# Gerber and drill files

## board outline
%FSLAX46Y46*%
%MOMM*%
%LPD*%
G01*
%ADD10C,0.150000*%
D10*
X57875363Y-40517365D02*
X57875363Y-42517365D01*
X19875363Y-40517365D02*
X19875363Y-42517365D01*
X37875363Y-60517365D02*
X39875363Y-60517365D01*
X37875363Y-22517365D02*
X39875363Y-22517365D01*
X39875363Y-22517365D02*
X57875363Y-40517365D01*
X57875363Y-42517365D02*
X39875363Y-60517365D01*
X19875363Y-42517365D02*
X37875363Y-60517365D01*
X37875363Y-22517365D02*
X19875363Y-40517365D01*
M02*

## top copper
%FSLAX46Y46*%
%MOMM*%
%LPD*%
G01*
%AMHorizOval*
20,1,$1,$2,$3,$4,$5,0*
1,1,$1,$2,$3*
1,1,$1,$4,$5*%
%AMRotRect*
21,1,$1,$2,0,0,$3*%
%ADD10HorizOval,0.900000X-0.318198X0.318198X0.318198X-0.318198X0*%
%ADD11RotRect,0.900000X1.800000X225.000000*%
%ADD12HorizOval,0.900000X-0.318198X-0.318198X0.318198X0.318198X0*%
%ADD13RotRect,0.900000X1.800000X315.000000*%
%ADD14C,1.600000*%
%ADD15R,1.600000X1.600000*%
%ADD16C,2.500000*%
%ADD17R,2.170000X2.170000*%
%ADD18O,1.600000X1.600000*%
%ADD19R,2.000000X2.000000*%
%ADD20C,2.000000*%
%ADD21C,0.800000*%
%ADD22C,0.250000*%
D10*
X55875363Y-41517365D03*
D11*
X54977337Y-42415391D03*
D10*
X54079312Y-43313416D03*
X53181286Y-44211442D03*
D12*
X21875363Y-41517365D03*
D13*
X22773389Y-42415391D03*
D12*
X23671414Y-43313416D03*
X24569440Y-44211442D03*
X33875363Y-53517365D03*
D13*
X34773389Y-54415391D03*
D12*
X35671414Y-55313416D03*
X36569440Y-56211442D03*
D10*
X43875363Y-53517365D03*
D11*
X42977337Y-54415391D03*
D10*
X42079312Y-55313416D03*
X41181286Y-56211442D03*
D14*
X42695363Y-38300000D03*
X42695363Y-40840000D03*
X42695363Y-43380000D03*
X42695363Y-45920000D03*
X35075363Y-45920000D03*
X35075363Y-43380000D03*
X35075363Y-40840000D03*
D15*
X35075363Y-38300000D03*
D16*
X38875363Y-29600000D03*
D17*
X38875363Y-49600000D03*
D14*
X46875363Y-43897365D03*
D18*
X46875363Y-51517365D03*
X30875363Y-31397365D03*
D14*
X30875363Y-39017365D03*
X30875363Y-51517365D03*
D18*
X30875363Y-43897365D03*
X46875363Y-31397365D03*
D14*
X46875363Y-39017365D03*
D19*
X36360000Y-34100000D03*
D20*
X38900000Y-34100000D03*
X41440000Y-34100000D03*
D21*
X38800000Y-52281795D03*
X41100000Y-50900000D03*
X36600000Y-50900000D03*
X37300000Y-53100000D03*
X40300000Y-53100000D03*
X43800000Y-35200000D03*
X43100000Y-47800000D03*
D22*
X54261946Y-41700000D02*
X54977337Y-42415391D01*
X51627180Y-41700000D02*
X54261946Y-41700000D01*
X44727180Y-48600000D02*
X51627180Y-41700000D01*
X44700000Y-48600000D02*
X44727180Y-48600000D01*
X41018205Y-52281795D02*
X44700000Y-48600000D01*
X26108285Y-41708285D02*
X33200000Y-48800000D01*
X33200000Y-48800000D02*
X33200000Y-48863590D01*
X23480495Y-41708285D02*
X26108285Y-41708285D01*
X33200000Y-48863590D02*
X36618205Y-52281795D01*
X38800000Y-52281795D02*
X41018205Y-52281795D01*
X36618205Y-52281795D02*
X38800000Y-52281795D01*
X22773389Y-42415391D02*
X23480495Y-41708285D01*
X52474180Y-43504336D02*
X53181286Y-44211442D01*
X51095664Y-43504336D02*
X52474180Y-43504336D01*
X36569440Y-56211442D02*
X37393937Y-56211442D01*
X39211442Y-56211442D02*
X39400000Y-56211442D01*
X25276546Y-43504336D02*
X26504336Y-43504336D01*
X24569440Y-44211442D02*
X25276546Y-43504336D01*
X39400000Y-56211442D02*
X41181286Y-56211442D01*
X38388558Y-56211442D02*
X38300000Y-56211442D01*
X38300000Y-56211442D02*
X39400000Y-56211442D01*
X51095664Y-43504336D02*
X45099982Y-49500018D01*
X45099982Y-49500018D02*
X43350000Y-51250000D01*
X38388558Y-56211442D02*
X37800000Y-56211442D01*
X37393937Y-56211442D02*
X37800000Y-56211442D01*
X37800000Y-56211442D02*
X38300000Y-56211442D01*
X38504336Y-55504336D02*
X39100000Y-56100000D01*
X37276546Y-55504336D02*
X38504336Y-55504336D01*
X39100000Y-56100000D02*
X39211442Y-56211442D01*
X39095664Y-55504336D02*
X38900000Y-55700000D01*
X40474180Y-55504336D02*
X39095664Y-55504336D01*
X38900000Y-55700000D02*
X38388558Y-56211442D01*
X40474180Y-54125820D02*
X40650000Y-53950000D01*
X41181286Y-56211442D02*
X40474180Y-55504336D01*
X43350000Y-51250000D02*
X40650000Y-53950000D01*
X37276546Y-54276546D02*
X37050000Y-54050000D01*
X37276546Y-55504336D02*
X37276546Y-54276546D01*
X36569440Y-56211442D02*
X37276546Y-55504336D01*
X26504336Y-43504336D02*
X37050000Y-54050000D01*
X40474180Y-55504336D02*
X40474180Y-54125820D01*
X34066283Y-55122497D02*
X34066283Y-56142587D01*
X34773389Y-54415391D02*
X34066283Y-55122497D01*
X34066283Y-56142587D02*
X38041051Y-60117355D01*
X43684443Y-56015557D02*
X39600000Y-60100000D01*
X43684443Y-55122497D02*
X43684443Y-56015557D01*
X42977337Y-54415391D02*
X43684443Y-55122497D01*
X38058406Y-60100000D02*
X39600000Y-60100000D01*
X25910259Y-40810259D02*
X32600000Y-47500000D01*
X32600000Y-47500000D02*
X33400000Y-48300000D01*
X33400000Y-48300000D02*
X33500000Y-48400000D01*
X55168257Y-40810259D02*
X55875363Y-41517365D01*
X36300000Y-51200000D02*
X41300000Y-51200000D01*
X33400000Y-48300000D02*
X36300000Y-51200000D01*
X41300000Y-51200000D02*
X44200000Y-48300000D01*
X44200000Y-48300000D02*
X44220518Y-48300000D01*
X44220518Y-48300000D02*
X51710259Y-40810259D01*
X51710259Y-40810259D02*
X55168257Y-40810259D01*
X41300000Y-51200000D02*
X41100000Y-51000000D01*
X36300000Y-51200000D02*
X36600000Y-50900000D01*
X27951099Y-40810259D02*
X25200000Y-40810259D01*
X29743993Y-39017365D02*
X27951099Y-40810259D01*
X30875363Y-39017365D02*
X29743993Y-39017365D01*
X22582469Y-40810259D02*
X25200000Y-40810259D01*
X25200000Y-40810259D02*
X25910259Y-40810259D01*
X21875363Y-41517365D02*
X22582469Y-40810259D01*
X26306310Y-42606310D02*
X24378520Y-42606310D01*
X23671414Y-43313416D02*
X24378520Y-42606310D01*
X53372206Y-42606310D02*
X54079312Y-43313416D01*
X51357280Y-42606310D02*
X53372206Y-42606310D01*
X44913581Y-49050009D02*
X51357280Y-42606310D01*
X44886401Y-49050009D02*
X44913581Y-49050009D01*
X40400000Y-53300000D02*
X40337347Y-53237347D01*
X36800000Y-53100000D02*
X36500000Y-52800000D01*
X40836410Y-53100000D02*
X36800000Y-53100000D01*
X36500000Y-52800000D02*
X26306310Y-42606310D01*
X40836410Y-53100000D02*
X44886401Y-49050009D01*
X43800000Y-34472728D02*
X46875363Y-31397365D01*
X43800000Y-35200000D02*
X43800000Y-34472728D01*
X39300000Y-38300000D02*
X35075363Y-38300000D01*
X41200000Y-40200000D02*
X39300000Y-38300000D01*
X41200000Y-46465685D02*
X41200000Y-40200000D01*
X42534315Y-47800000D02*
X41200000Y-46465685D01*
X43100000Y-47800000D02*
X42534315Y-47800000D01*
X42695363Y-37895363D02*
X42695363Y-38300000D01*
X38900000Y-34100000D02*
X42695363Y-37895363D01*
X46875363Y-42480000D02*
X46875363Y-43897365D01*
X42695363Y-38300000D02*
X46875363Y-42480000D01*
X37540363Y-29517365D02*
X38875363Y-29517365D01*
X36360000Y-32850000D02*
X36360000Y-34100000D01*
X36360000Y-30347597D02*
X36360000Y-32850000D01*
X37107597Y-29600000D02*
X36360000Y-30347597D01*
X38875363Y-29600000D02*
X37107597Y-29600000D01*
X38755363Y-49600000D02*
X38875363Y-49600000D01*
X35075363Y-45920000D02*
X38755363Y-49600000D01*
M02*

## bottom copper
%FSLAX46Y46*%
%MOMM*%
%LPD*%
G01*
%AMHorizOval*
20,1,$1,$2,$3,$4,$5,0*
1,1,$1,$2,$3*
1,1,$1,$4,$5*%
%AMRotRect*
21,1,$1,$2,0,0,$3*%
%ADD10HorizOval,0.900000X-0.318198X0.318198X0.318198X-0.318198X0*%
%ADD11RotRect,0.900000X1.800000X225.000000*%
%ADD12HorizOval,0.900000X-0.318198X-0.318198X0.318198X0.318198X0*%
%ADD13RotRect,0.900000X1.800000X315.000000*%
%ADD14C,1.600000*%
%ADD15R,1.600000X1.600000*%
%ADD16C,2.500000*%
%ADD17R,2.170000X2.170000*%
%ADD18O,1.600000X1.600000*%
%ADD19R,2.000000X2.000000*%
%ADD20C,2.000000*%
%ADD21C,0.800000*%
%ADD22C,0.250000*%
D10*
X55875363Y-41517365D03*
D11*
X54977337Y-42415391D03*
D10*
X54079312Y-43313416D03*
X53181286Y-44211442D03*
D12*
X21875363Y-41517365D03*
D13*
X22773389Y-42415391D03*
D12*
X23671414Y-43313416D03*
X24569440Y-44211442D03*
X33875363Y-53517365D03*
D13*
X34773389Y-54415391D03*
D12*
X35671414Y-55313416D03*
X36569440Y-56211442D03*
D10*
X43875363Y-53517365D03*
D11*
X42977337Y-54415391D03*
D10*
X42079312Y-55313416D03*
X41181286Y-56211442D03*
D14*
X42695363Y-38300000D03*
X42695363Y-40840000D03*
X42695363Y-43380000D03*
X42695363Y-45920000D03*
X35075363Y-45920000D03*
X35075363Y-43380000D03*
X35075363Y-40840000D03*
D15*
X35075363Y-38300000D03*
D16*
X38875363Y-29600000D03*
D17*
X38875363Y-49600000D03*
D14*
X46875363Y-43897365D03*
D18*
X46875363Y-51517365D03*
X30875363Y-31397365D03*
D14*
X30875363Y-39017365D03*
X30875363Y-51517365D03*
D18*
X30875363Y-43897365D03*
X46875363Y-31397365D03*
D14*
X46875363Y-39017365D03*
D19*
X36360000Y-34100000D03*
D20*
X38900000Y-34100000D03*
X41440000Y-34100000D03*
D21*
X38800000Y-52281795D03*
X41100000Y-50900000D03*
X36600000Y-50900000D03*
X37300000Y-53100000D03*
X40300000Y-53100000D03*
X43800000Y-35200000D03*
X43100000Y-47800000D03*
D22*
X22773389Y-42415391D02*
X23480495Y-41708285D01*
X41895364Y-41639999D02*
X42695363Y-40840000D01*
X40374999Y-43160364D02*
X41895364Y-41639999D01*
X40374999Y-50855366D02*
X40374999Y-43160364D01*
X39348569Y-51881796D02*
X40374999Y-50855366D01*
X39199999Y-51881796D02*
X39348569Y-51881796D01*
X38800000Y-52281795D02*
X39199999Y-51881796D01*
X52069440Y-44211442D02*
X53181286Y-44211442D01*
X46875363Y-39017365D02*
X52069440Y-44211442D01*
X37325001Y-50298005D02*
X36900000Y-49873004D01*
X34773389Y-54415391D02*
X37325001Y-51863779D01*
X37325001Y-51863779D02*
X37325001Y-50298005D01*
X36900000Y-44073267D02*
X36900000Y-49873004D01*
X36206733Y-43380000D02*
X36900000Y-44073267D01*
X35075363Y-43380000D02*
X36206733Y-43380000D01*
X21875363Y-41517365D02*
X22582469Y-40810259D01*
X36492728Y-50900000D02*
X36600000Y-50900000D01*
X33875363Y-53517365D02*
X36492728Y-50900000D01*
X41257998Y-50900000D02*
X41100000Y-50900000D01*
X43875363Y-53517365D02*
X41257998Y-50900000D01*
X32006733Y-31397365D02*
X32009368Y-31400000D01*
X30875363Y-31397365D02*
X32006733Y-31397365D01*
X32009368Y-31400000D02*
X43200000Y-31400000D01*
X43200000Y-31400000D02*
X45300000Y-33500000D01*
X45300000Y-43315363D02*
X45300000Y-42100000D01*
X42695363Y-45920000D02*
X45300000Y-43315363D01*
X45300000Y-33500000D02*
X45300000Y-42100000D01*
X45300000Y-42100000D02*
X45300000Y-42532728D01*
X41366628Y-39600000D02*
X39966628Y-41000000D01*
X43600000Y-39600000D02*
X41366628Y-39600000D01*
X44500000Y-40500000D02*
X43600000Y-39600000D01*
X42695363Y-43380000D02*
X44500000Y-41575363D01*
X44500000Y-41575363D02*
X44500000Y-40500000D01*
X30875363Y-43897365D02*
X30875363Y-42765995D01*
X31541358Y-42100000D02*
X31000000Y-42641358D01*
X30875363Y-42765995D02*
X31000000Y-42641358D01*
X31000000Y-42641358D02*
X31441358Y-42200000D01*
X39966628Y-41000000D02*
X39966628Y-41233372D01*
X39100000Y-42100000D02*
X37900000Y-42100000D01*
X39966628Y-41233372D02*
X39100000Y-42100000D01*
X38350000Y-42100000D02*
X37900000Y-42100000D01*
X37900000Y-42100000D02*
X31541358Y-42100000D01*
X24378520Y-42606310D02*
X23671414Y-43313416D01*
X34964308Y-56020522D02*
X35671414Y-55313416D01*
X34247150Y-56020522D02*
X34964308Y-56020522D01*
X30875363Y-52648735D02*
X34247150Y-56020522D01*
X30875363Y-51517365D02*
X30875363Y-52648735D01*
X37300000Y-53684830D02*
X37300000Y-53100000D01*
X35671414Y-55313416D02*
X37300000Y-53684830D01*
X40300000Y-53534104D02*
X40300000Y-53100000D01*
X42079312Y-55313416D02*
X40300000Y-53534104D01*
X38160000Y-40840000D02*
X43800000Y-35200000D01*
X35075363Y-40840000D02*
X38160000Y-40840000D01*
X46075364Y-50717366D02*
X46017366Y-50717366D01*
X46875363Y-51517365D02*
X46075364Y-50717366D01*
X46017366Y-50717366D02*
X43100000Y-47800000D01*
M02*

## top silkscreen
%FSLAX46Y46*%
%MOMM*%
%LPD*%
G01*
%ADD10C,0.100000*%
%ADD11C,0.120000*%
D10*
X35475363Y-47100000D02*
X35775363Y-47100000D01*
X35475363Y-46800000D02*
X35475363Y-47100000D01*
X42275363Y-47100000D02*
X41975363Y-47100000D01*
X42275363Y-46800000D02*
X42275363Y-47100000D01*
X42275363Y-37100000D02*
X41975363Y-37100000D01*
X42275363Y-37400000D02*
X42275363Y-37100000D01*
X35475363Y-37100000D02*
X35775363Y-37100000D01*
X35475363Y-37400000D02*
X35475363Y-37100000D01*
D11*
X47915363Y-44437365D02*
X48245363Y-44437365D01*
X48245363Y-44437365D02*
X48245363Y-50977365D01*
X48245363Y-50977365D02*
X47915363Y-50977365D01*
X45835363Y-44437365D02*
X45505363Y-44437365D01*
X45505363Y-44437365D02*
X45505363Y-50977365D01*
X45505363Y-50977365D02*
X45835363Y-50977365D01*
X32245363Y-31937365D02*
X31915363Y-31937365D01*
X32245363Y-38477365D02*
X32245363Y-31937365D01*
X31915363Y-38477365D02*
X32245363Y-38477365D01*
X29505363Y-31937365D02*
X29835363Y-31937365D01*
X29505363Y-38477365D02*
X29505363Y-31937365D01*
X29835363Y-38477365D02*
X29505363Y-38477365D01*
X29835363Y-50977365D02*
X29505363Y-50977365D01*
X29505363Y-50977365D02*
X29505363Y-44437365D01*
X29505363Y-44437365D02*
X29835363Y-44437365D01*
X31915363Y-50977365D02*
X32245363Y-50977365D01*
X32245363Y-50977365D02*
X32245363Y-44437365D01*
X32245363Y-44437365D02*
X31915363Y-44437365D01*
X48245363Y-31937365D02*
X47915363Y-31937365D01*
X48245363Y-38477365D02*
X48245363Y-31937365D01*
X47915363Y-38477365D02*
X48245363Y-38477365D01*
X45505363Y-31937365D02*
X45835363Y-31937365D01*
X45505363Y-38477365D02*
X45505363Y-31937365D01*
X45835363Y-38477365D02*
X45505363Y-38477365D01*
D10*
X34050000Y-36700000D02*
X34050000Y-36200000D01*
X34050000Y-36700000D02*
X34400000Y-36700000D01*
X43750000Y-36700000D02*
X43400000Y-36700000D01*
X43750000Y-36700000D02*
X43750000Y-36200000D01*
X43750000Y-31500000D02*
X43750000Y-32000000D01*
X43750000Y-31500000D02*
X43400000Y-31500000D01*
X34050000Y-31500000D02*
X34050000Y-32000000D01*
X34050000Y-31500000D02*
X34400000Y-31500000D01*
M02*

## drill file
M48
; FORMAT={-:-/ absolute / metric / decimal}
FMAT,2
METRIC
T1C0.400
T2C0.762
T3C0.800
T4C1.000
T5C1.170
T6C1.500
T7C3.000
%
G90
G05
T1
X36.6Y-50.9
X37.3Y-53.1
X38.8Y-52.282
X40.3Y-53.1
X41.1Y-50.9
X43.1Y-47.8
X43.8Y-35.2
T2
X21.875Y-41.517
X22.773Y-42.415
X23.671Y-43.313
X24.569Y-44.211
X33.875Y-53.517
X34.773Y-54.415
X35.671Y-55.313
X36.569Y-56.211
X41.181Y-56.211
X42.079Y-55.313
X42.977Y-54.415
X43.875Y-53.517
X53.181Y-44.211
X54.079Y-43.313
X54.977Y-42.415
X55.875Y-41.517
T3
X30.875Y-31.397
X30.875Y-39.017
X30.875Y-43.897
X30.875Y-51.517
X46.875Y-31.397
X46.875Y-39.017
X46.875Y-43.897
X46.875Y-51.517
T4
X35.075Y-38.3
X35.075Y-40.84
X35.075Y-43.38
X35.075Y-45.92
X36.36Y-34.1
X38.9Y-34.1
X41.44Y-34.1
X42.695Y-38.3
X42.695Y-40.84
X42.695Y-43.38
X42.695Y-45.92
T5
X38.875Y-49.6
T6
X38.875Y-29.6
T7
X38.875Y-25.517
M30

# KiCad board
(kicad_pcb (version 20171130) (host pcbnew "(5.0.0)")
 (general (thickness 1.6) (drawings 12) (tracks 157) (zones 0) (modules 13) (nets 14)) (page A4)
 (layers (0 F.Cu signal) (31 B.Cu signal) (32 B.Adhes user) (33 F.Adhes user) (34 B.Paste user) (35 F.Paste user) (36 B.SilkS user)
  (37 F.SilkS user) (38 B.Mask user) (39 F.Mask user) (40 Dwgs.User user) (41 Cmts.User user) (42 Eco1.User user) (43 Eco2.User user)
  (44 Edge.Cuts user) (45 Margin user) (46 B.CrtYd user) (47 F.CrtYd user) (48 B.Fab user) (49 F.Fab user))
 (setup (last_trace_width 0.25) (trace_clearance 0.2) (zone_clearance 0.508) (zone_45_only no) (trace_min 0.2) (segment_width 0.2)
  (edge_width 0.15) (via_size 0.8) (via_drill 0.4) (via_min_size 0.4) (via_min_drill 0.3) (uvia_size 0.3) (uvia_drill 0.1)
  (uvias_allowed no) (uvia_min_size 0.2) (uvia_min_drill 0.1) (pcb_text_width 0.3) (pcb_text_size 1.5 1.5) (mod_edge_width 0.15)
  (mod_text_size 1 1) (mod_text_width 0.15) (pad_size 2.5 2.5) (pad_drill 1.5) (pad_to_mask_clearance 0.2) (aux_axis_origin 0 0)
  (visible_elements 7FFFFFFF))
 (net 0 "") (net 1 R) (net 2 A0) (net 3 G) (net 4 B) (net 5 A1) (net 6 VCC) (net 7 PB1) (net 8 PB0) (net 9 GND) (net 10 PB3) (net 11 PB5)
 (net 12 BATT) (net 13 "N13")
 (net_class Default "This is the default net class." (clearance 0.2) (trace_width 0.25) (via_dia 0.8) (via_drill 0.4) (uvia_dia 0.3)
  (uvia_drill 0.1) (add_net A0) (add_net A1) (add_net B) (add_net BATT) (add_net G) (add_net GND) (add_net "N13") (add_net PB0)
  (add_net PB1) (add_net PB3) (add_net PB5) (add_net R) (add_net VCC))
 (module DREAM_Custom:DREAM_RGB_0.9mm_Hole (layer F.Cu) (at 55.875363 41.517365 225)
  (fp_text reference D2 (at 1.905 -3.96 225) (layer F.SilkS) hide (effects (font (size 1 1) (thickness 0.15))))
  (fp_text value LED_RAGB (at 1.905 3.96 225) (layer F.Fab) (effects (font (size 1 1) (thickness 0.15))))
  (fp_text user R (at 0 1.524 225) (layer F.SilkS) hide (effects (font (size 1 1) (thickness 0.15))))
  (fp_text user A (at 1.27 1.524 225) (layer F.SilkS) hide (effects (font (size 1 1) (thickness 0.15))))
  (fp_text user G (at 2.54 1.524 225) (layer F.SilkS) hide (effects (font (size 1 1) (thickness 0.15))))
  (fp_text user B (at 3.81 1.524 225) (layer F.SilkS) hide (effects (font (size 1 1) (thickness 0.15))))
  (pad 1 thru_hole oval (at 0 0 225) (size 0.9 1.8) (drill 0.762) (layers *.Cu *.Mask) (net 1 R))
  (pad 2 thru_hole rect (at 1.270001 0 225) (size 0.9 1.8) (drill 0.762) (layers *.Cu *.Mask) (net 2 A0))
  (pad 3 thru_hole oval (at 2.54 0 225) (size 0.9 1.8) (drill 0.762) (layers *.Cu *.Mask) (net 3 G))
  (pad 4 thru_hole oval (at 3.81 0 225) (size 0.9 1.8) (drill 0.762) (layers *.Cu *.Mask) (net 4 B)))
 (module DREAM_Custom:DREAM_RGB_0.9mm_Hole (layer F.Cu) (at 21.875363 41.517365 315)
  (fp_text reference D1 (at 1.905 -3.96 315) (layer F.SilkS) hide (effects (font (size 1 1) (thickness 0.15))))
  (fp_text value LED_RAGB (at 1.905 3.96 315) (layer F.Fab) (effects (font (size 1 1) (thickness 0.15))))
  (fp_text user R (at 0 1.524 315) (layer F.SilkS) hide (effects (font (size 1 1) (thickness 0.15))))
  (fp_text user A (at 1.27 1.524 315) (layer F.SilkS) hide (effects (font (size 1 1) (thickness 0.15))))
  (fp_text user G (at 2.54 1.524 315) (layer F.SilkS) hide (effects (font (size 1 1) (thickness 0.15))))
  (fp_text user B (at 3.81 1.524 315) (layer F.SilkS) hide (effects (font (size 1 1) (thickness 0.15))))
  (pad 1 thru_hole oval (at 0 0 315) (size 0.9 1.8) (drill 0.762) (layers *.Cu *.Mask) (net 1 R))
  (pad 2 thru_hole rect (at 1.270001 0 315) (size 0.9 1.8) (drill 0.762) (layers *.Cu *.Mask) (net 2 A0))
  (pad 3 thru_hole oval (at 2.54 0 315) (size 0.9 1.8) (drill 0.762) (layers *.Cu *.Mask) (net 3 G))
  (pad 4 thru_hole oval (at 3.81 0 315) (size 0.9 1.8) (drill 0.762) (layers *.Cu *.Mask) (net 4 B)))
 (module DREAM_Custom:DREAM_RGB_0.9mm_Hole (layer F.Cu) (at 33.875363 53.517365 315)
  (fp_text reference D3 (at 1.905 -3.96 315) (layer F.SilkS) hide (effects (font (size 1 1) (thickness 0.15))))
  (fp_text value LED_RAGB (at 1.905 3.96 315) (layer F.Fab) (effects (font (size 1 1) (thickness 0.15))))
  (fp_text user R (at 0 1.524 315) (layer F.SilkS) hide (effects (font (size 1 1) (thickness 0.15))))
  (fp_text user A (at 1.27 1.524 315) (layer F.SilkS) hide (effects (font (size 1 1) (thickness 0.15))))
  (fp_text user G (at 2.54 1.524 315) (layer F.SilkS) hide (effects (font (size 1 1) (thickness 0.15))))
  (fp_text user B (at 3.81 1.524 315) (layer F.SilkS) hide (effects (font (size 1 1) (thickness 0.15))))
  (pad 1 thru_hole oval (at 0 0 315) (size 0.9 1.8) (drill 0.762) (layers *.Cu *.Mask) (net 1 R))
  (pad 2 thru_hole rect (at 1.270001 0 315) (size 0.9 1.8) (drill 0.762) (layers *.Cu *.Mask) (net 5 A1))
  (pad 3 thru_hole oval (at 2.54 0 315) (size 0.9 1.8) (drill 0.762) (layers *.Cu *.Mask) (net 3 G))
  (pad 4 thru_hole oval (at 3.81 0 315) (size 0.9 1.8) (drill 0.762) (layers *.Cu *.Mask) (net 4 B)))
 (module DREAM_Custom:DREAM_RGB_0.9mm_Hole (layer F.Cu) (at 43.875363 53.517365 225)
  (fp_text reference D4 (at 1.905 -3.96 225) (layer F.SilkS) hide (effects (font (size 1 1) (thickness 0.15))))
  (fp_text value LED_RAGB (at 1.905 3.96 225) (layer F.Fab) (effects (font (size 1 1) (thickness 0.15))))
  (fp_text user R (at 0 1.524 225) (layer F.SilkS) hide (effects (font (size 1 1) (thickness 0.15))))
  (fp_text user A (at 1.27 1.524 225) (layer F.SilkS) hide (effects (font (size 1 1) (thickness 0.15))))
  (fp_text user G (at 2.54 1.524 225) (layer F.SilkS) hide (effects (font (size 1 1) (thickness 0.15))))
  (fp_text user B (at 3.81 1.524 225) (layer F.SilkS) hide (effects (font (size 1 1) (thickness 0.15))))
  (pad 1 thru_hole oval (at 0 0 225) (size 0.9 1.8) (drill 0.762) (layers *.Cu *.Mask) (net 1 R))
  (pad 2 thru_hole rect (at 1.270001 0 225) (size 0.9 1.8) (drill 0.762) (layers *.Cu *.Mask) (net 5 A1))
  (pad 3 thru_hole oval (at 2.54 0 225) (size 0.9 1.8) (drill 0.762) (layers *.Cu *.Mask) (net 3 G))
  (pad 4 thru_hole oval (at 3.81 0 225) (size 0.9 1.8) (drill 0.762) (layers *.Cu *.Mask) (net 4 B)))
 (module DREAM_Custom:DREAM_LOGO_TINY (layer B.Cu) (at 38.9 40.65 180)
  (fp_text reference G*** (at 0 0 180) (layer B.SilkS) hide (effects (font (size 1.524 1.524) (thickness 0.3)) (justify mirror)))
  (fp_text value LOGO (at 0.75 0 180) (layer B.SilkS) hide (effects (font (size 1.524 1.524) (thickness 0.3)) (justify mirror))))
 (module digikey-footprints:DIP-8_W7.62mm (layer F.Cu) (at 35.075363 38.3)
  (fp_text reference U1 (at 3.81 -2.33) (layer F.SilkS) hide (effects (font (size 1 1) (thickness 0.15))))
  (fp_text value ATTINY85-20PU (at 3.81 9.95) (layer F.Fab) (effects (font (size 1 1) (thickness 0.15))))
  (fp_line (start 0.4 8.8) (end 0.7 8.8) (layer F.SilkS) (width 0.1))
  (fp_line (start 0.4 8.5) (end 0.4 8.8) (layer F.SilkS) (width 0.1))
  (fp_line (start 7.2 8.8) (end 6.9 8.8) (layer F.SilkS) (width 0.1))
  (fp_line (start 7.2 8.5) (end 7.2 8.8) (layer F.SilkS) (width 0.1))
  (fp_line (start 7.2 -1.2) (end 6.9 -1.2) (layer F.SilkS) (width 0.1))
  (fp_line (start 7.2 -0.9) (end 7.2 -1.2) (layer F.SilkS) (width 0.1))
  (fp_line (start 0.4 -1.2) (end 0.7 -1.2) (layer F.SilkS) (width 0.1))
  (fp_line (start 0.4 -0.9) (end 0.4 -1.2) (layer F.SilkS) (width 0.1))
  (pad 8 thru_hole circle (at 7.62 0) (size 1.6 1.6) (drill 1) (layers *.Cu *.Mask) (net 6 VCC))
  (pad 7 thru_hole circle (at 7.62 2.54) (size 1.6 1.6) (drill 1) (layers *.Cu *.Mask) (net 2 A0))
  (pad 6 thru_hole circle (at 7.62 5.08) (size 1.6 1.6) (drill 1) (layers *.Cu *.Mask) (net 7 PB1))
  (pad 5 thru_hole circle (at 7.62 7.62) (size 1.6 1.6) (drill 1) (layers *.Cu *.Mask) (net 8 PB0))
  (pad 4 thru_hole circle (at 0 7.62) (size 1.6 1.6) (drill 1) (layers *.Cu *.Mask) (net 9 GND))
  (pad 3 thru_hole circle (at 0 5.08) (size 1.6 1.6) (drill 1) (layers *.Cu *.Mask) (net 5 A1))
  (pad 2 thru_hole circle (at 0 2.54) (size 1.6 1.6) (drill 1) (layers *.Cu *.Mask) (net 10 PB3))
  (pad 1 thru_hole rect (at 0 0) (size 1.6 1.6) (drill 1) (layers *.Cu *.Mask) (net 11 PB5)))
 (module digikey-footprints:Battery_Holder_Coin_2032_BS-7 (layer B.Cu) (at 38.875363 49.6 90)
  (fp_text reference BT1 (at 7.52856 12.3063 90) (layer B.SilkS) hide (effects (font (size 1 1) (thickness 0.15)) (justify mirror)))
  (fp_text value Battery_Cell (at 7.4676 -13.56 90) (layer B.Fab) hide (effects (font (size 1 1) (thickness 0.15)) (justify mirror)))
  (pad Pos thru_hole circle (at 20 0 90) (size 2.5 2.5) (drill 1.5) (layers *.Cu *.Mask) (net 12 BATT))
  (pad Neg thru_hole rect (at 0 0 90) (size 2.17 2.17) (drill 1.17) (layers *.Cu *.Mask) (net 9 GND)))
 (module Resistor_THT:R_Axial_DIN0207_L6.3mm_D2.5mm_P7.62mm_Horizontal (layer F.Cu) (at 46.875363 43.897365 270)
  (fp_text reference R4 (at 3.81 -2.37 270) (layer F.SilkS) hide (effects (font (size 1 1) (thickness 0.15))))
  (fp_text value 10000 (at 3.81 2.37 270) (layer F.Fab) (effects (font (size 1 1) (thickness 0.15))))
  (fp_line (start 0.54 -1.04) (end 0.54 -1.37) (layer F.SilkS) (width 0.12))
  (fp_line (start 0.54 -1.37) (end 7.08 -1.37) (layer F.SilkS) (width 0.12))
  (fp_line (start 7.08 -1.37) (end 7.08 -1.04) (layer F.SilkS) (width 0.12))
  (fp_line (start 0.54 1.04) (end 0.54 1.37) (layer F.SilkS) (width 0.12))
  (fp_line (start 0.54 1.37) (end 7.08 1.37) (layer F.SilkS) (width 0.12))
  (fp_line (start 7.08 1.37) (end 7.08 1.04) (layer F.SilkS) (width 0.12))
  (pad 1 thru_hole circle (at 0 0 270) (size 1.6 1.6) (drill 0.8) (layers *.Cu *.Mask) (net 6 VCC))
  (pad 2 thru_hole oval (at 7.62 0 270) (size 1.6 1.6) (drill 0.8) (layers *.Cu *.Mask) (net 11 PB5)))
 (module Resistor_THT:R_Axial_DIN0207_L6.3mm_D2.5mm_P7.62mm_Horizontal (layer F.Cu) (at 30.875363 39.017365 90)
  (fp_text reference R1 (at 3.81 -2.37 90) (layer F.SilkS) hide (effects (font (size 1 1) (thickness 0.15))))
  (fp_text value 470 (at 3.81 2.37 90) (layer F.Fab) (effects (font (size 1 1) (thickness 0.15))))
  (fp_line (start 7.08 1.37) (end 7.08 1.04) (layer F.SilkS) (width 0.12))
  (fp_line (start 0.54 1.37) (end 7.08 1.37) (layer F.SilkS) (width 0.12))
  (fp_line (start 0.54 1.04) (end 0.54 1.37) (layer F.SilkS) (width 0.12))
  (fp_line (start 7.08 -1.37) (end 7.08 -1.04) (layer F.SilkS) (width 0.12))
  (fp_line (start 0.54 -1.37) (end 7.08 -1.37) (layer F.SilkS) (width 0.12))
  (fp_line (start 0.54 -1.04) (end 0.54 -1.37) (layer F.SilkS) (width 0.12))
  (pad 2 thru_hole oval (at 7.62 0 90) (size 1.6 1.6) (drill 0.8) (layers *.Cu *.Mask) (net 8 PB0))
  (pad 1 thru_hole circle (at 0 0 90) (size 1.6 1.6) (drill 0.8) (layers *.Cu *.Mask) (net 1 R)))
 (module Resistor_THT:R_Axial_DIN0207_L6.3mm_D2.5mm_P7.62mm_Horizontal (layer F.Cu) (at 30.875363 51.517365 90)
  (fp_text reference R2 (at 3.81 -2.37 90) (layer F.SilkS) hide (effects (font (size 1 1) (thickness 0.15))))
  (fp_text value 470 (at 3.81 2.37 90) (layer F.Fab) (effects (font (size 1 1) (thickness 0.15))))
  (fp_line (start 0.54 -1.04) (end 0.54 -1.37) (layer F.SilkS) (width 0.12))
  (fp_line (start 0.54 -1.37) (end 7.08 -1.37) (layer F.SilkS) (width 0.12))
  (fp_line (start 7.08 -1.37) (end 7.08 -1.04) (layer F.SilkS) (width 0.12))
  (fp_line (start 0.54 1.04) (end 0.54 1.37) (layer F.SilkS) (width 0.12))
  (fp_line (start 0.54 1.37) (end 7.08 1.37) (layer F.SilkS) (width 0.12))
  (fp_line (start 7.08 1.37) (end 7.08 1.04) (layer F.SilkS) (width 0.12))
  (pad 1 thru_hole circle (at 0 0 90) (size 1.6 1.6) (drill 0.8) (layers *.Cu *.Mask) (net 3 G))
  (pad 2 thru_hole oval (at 7.62 0 90) (size 1.6 1.6) (drill 0.8) (layers *.Cu *.Mask) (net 7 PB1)))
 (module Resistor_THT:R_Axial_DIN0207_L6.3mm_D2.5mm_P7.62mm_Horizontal (layer F.Cu) (at 46.875363 39.017365 90)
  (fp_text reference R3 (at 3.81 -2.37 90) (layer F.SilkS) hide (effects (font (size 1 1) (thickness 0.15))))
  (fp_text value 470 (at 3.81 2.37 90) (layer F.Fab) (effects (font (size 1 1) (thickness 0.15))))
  (fp_line (start 7.08 1.37) (end 7.08 1.04) (layer F.SilkS) (width 0.12))
  (fp_line (start 0.54 1.37) (end 7.08 1.37) (layer F.SilkS) (width 0.12))
  (fp_line (start 0.54 1.04) (end 0.54 1.37) (layer F.SilkS) (width 0.12))
  (fp_line (start 7.08 -1.37) (end 7.08 -1.04) (layer F.SilkS) (width 0.12))
  (fp_line (start 0.54 -1.37) (end 7.08 -1.37) (layer F.SilkS) (width 0.12))
  (fp_line (start 0.54 -1.04) (end 0.54 -1.37) (layer F.SilkS) (width 0.12))
  (pad 2 thru_hole oval (at 7.62 0 90) (size 1.6 1.6) (drill 0.8) (layers *.Cu *.Mask) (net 10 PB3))
  (pad 1 thru_hole circle (at 0 0 90) (size 1.6 1.6) (drill 0.8) (layers *.Cu *.Mask) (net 4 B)))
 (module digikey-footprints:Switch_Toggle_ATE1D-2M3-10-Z (layer F.Cu) (at 38.9 34.1)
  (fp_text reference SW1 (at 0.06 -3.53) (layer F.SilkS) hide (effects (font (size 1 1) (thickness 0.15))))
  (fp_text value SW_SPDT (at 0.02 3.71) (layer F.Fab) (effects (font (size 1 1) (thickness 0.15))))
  (fp_line (start -4.85 2.6) (end -4.85 2.1) (layer F.SilkS) (width 0.1))
  (fp_line (start -4.85 2.6) (end -4.5 2.6) (layer F.SilkS) (width 0.1))
  (fp_line (start 4.85 2.6) (end 4.5 2.6) (layer F.SilkS) (width 0.1))
  (fp_line (start 4.85 2.6) (end 4.85 2.1) (layer F.SilkS) (width 0.1))
  (fp_line (start 4.85 -2.6) (end 4.85 -2.1) (layer F.SilkS) (width 0.1))
  (fp_line (start 4.85 -2.6) (end 4.5 -2.6) (layer F.SilkS) (width 0.1))
  (fp_line (start -4.85 -2.6) (end -4.85 -2.1) (layer F.SilkS) (width 0.1))
  (fp_line (start -4.85 -2.6) (end -4.5 -2.6) (layer F.SilkS) (width 0.1))
  (pad 1 thru_hole rect (at -2.54 0) (size 2 2) (drill 1) (layers *.Cu *.Mask) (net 12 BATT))
  (pad 2 thru_hole circle (at 0 0) (size 2 2) (drill 1) (layers *.Cu *.Mask) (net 6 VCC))
  (pad 3 thru_hole circle (at 2.54 0) (size 2 2) (drill 1) (layers *.Cu *.Mask) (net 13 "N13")))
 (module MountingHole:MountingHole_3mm (layer F.Cu) (at 38.875363 25.517365)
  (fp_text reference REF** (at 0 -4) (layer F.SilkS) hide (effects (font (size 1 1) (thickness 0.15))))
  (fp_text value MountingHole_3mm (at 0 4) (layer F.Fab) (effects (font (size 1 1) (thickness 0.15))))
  (pad 1 np_thru_hole circle (at 0 0) (size 3 3) (drill 3) (layers *.Cu *.Mask)))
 (gr_line (start 57.875363 40.517365) (end 57.875363 42.517365) (layer Edge.Cuts) (width 0.15))
 (gr_line (start 19.875363 40.517365) (end 19.875363 42.517365) (layer Edge.Cuts) (width 0.15))
 (gr_line (start 37.875363 60.517365) (end 39.875363 60.517365) (layer Edge.Cuts) (width 0.15))
 (gr_line (start 37.875363 22.517365) (end 39.875363 22.517365) (layer Edge.Cuts) (width 0.15))
 (gr_line (start 39.875363 22.517365) (end 57.875363 40.517365) (layer Edge.Cuts) (width 0.15))
 (gr_line (start 57.875363 42.517365) (end 39.875363 60.517365) (layer Edge.Cuts) (width 0.15))
 (gr_line (start 19.875363 42.517365) (end 37.875363 60.517365) (layer Edge.Cuts) (width 0.15))
 (gr_line (start 37.875363 22.517365) (end 19.875363 40.517365) (layer Edge.Cuts) (width 0.15))
 (segment (start 54.261946 41.7) (end 54.977337 42.415391) (width 0.25) (layer F.Cu) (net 2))
 (segment (start 51.62718 41.7) (end 54.261946 41.7) (width 0.25) (layer F.Cu) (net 2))
 (segment (start 44.72718 48.6) (end 51.62718 41.7) (width 0.25) (layer F.Cu) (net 2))
 (segment (start 44.7 48.6) (end 44.72718 48.6) (width 0.25) (layer F.Cu) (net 2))
 (segment (start 41.018205 52.281795) (end 44.7 48.6) (width 0.25) (layer F.Cu) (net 2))
 (segment (start 22.773389 42.415391) (end 23.480495 41.708285) (width 0.25) (layer B.Cu) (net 2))
 (segment (start 26.108285 41.708285) (end 33.2 48.8) (width 0.25) (layer F.Cu) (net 2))
 (segment (start 33.2 48.8) (end 33.2 48.86359) (width 0.25) (layer F.Cu) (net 2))
 (segment (start 23.480495 41.708285) (end 26.108285 41.708285) (width 0.25) (layer F.Cu) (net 2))
 (segment (start 33.2 48.86359) (end 36.618205 52.281795) (width 0.25) (layer F.Cu) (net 2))
 (via (at 38.8 52.281795) (size 0.8) (drill 0.4) (layers F.Cu B.Cu) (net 2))
 (segment (start 38.8 52.281795) (end 41.018205 52.281795) (width 0.25) (layer F.Cu) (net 2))
 (segment (start 36.618205 52.281795) (end 38.8 52.281795) (width 0.25) (layer F.Cu) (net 2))
 (segment (start 22.773389 42.415391) (end 23.480495 41.708285) (width 0.25) (layer F.Cu) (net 2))
 (segment (start 41.895364 41.639999) (end 42.695363 40.84) (width 0.25) (layer B.Cu) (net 2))
 (segment (start 40.374999 43.160364) (end 41.895364 41.639999) (width 0.25) (layer B.Cu) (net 2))
 (segment (start 40.374999 50.855366) (end 40.374999 43.160364) (width 0.25) (layer B.Cu) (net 2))
 (segment (start 39.348569 51.881796) (end 40.374999 50.855366) (width 0.25) (layer B.Cu) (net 2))
 (segment (start 39.199999 51.881796) (end 39.348569 51.881796) (width 0.25) (layer B.Cu) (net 2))
 (segment (start 38.8 52.281795) (end 39.199999 51.881796) (width 0.25) (layer B.Cu) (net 2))
 (segment (start 52.06944 44.211442) (end 53.181286 44.211442) (width 0.25) (layer B.Cu) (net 4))
 (segment (start 46.875363 39.017365) (end 52.06944 44.211442) (width 0.25) (layer B.Cu) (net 4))
 (segment (start 52.47418 43.504336) (end 53.181286 44.211442) (width 0.25) (layer F.Cu) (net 4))
 (segment (start 51.095664 43.504336) (end 52.47418 43.504336) (width 0.25) (layer F.Cu) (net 4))
 (segment (start 36.56944 56.211442) (end 37.393937 56.211442) (width 0.25) (layer F.Cu) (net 4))
 (segment (start 39.211442 56.211442) (end 39.4 56.211442) (width 0.25) (layer F.Cu) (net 4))
 (segment (start 25.276546 43.504336) (end 26.504336 43.504336) (width 0.25) (layer F.Cu) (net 4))
 (segment (start 24.56944 44.211442) (end 25.276546 43.504336) (width 0.25) (layer F.Cu) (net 4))
 (segment (start 39.4 56.211442) (end 41.181286 56.211442) (width 0.25) (layer F.Cu) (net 4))
 (segment (start 38.388558 56.211442) (end 38.3 56.211442) (width 0.25) (layer F.Cu) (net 4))
 (segment (start 38.3 56.211442) (end 39.4 56.211442) (width 0.25) (layer F.Cu) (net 4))
 (segment (start 51.095664 43.504336) (end 45.099982 49.500018) (width 0.25) (layer F.Cu) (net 4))
 (segment (start 45.099982 49.500018) (end 43.35 51.25) (width 0.25) (layer F.Cu) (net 4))
 (segment (start 38.388558 56.211442) (end 37.8 56.211442) (width 0.25) (layer F.Cu) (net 4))
 (segment (start 37.393937 56.211442) (end 37.8 56.211442) (width 0.25) (layer F.Cu) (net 4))
 (segment (start 37.8 56.211442) (end 38.3 56.211442) (width 0.25) (layer F.Cu) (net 4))
 (segment (start 38.504336 55.504336) (end 39.1 56.1) (width 0.25) (layer F.Cu) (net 4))
 (segment (start 37.276546 55.504336) (end 38.504336 55.504336) (width 0.25) (layer F.Cu) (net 4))
 (segment (start 39.1 56.1) (end 39.211442 56.211442) (width 0.25) (layer F.Cu) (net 4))
 (segment (start 39.095664 55.504336) (end 38.9 55.7) (width 0.25) (layer F.Cu) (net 4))
 (segment (start 40.47418 55.504336) (end 39.095664 55.504336) (width 0.25) (layer F.Cu) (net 4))
 (segment (start 38.9 55.7) (end 38.388558 56.211442) (width 0.25) (layer F.Cu) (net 4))
 (segment (start 40.47418 54.12582) (end 40.65 53.95) (width 0.25) (layer F.Cu) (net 4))
 (segment (start 41.181286 56.211442) (end 40.47418 55.504336) (width 0.25) (layer F.Cu) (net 4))
 (segment (start 43.35 51.25) (end 40.65 53.95) (width 0.25) (layer F.Cu) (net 4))
 (segment (start 37.276546 54.276546) (end 37.05 54.05) (width 0.25) (layer F.Cu) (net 4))
 (segment (start 37.276546 55.504336) (end 37.276546 54.276546) (width 0.25) (layer F.Cu) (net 4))
 (segment (start 36.56944 56.211442) (end 37.276546 55.504336) (width 0.25) (layer F.Cu) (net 4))
 (segment (start 26.504336 43.504336) (end 37.05 54.05) (width 0.25) (layer F.Cu) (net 4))
 (segment (start 40.47418 55.504336) (end 40.47418 54.12582) (width 0.25) (layer F.Cu) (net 4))
 (segment (start 34.066283 55.122497) (end 34.066283 56.142587) (width 0.25) (layer F.Cu) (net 5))
 (segment (start 34.773389 54.415391) (end 34.066283 55.122497) (width 0.25) (layer F.Cu) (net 5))
 (segment (start 34.066283 56.142587) (end 38.041051 60.117355) (width 0.25) (layer F.Cu) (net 5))
 (segment (start 43.684443 56.015557) (end 39.6 60.1) (width 0.25) (layer F.Cu) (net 5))
 (segment (start 43.684443 55.122497) (end 43.684443 56.015557) (width 0.25) (layer F.Cu) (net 5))
 (segment (start 42.977337 54.415391) (end 43.684443 55.122497) (width 0.25) (layer F.Cu) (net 5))
 (segment (start 38.058406 60.1) (end 39.6 60.1) (width 0.25) (layer F.Cu) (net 5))
 (segment (start 37.325001 50.298005) (end 36.9 49.873004) (width 0.25) (layer B.Cu) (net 5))
 (segment (start 34.773389 54.415391) (end 37.325001 51.863779) (width 0.25) (layer B.Cu) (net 5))
 (segment (start 37.325001 51.863779) (end 37.325001 50.298005) (width 0.25) (layer B.Cu) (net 5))
 (segment (start 36.9 44.073267) (end 36.9 49.873004) (width 0.25) (layer B.Cu) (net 5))
 (segment (start 36.206733 43.38) (end 36.9 44.073267) (width 0.25) (layer B.Cu) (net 5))
 (segment (start 35.075363 43.38) (end 36.206733 43.38) (width 0.25) (layer B.Cu) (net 5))
 (segment (start 21.875363 41.517365) (end 22.582469 40.810259) (width 0.25) (layer B.Cu) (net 1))
 (segment (start 25.910259 40.810259) (end 32.6 47.5) (width 0.25) (layer F.Cu) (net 1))
 (segment (start 32.6 47.5) (end 33.4 48.3) (width 0.25) (layer F.Cu) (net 1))
 (segment (start 33.4 48.3) (end 33.5 48.4) (width 0.25) (layer F.Cu) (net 1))
 (segment (start 55.168257 40.810259) (end 55.875363 41.517365) (width 0.25) (layer F.Cu) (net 1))
 (segment (start 36.3 51.2) (end 41.3 51.2) (width 0.25) (layer F.Cu) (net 1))
 (segment (start 33.4 48.3) (end 36.3 51.2) (width 0.25) (layer F.Cu) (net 1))
 (segment (start 41.3 51.2) (end 44.2 48.3) (width 0.25) (layer F.Cu) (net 1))
 (segment (start 44.2 48.3) (end 44.220518 48.3) (width 0.25) (layer F.Cu) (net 1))
 (segment (start 44.220518 48.3) (end 51.710259 40.810259) (width 0.25) (layer F.Cu) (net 1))
 (segment (start 51.710259 40.810259) (end 55.168257 40.810259) (width 0.25) (layer F.Cu) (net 1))
 (via (at 41.1 50.9) (size 0.8) (drill 0.4) (layers F.Cu B.Cu) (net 1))
 (segment (start 41.3 51.2) (end 41.1 51) (width 0.25) (layer F.Cu) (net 1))
 (via (at 36.6 50.9) (size 0.8) (drill 0.4) (layers F.Cu B.Cu) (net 1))
 (segment (start 36.3 51.2) (end 36.6 50.9) (width 0.25) (layer F.Cu) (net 1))
 (segment (start 36.492728 50.9) (end 36.6 50.9) (width 0.25) (layer B.Cu) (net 1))
 (segment (start 33.875363 53.517365) (end 36.492728 50.9) (width 0.25) (layer B.Cu) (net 1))
 (segment (start 41.257998 50.9) (end 41.1 50.9) (width 0.25) (layer B.Cu) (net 1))
 (segment (start 43.875363 53.517365) (end 41.257998 50.9) (width 0.25) (layer B.Cu) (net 1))
 (segment (start 27.951099 40.810259) (end 25.2 40.810259) (width 0.25) (layer F.Cu) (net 1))
 (segment (start 29.743993 39.017365) (end 27.951099 40.810259) (width 0.25) (layer F.Cu) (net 1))
 (segment (start 30.875363 39.017365) (end 29.743993 39.017365) (width 0.25) (layer F.Cu) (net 1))
 (segment (start 22.582469 40.810259) (end 25.2 40.810259) (width 0.25) (layer F.Cu) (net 1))
 (segment (start 25.2 40.810259) (end 25.910259 40.810259) (width 0.25) (layer F.Cu) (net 1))
 (segment (start 21.875363 41.517365) (end 22.582469 40.810259) (width 0.25) (layer F.Cu) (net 1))
 (segment (start 32.006733 31.397365) (end 32.009368 31.4) (width 0.25) (layer B.Cu) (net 8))
 (segment (start 30.875363 31.397365) (end 32.006733 31.397365) (width 0.25) (layer B.Cu) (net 8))
 (segment (start 32.009368 31.4) (end 43.2 31.4) (width 0.25) (layer B.Cu) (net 8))
 (segment (start 43.2 31.4) (end 45.3 33.5) (width 0.25) (layer B.Cu) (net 8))
 (segment (start 45.3 43.315363) (end 45.3 42.1) (width 0.25) (layer B.Cu) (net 8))
 (segment (start 42.695363 45.92) (end 45.3 43.315363) (width 0.25) (layer B.Cu) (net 8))
 (segment (start 45.3 33.5) (end 45.3 42.1) (width 0.25) (layer B.Cu) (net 8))
 (segment (start 45.3 42.1) (end 45.3 42.532728) (width 0.25) (layer B.Cu) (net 8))
 (segment (start 41.366628 39.6) (end 39.966628 41) (width 0.25) (layer B.Cu) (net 7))
 (segment (start 43.6 39.6) (end 41.366628 39.6) (width 0.25) (layer B.Cu) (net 7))
 (segment (start 44.5 40.5) (end 43.6 39.6) (width 0.25) (layer B.Cu) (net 7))
 (segment (start 42.695363 43.38) (end 44.5 41.575363) (width 0.25) (layer B.Cu) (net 7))
 (segment (start 44.5 41.575363) (end 44.5 40.5) (width 0.25) (layer B.Cu) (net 7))
 (segment (start 30.875363 43.897365) (end 30.875363 42.765995) (width 0.25) (layer B.Cu) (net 7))
 (segment (start 31.541358 42.1) (end 31 42.641358) (width 0.25) (layer B.Cu) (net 7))
 (segment (start 30.875363 42.765995) (end 31 42.641358) (width 0.25) (layer B.Cu) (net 7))
 (segment (start 31 42.641358) (end 31.441358 42.2) (width 0.25) (layer B.Cu) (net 7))
 (segment (start 39.966628 41) (end 39.966628 41.233372) (width 0.25) (layer B.Cu) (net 7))
 (segment (start 39.1 42.1) (end 37.9 42.1) (width 0.25) (layer B.Cu) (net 7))
 (segment (start 39.966628 41.233372) (end 39.1 42.1) (width 0.25) (layer B.Cu) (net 7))
 (segment (start 38.35 42.1) (end 37.9 42.1) (width 0.25) (layer B.Cu) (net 7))
 (segment (start 37.9 42.1) (end 31.541358 42.1) (width 0.25) (layer B.Cu) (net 7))
 (segment (start 24.37852 42.60631) (end 23.671414 43.313416) (width 0.25) (layer B.Cu) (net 3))
 (segment (start 26.30631 42.60631) (end 24.37852 42.60631) (width 0.25) (layer F.Cu) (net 3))
 (via (at 37.3 53.1) (size 0.8) (drill 0.4) (layers F.Cu B.Cu) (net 3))
 (segment (start 34.964308 56.020522) (end 35.671414 55.313416) (width 0.25) (layer B.Cu) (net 3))
 (segment (start 34.24715 56.020522) (end 34.964308 56.020522) (width 0.25) (layer B.Cu) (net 3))
 (segment (start 30.875363 52.648735) (end 34.24715 56.020522) (width 0.25) (layer B.Cu) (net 3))
 (segment (start 30.875363 51.517365) (end 30.875363 52.648735) (width 0.25) (layer B.Cu) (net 3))
 (segment (start 23.671414 43.313416) (end 24.37852 42.60631) (width 0.25) (layer F.Cu) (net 3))
 (segment (start 53.372206 42.60631) (end 54.079312 43.313416) (width 0.25) (layer F.Cu) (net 3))
 (segment (start 51.35728 42.60631) (end 53.372206 42.60631) (width 0.25) (layer F.Cu) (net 3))
 (segment (start 44.913581 49.050009) (end 51.35728 42.60631) (width 0.25) (layer F.Cu) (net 3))
 (segment (start 44.886401 49.050009) (end 44.913581 49.050009) (width 0.25) (layer F.Cu) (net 3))
 (via (at 40.3 53.1) (size 0.8) (drill 0.4) (layers F.Cu B.Cu) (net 3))
 (segment (start 40.4 53.3) (end 40.337347 53.237347) (width 0.25) (layer F.Cu) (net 3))
 (segment (start 36.8 53.1) (end 36.5 52.8) (width 0.25) (layer F.Cu) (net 3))
 (segment (start 40.83641 53.1) (end 36.8 53.1) (width 0.25) (layer F.Cu) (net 3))
 (segment (start 36.5 52.8) (end 26.30631 42.60631) (width 0.25) (layer F.Cu) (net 3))
 (segment (start 40.83641 53.1) (end 44.886401 49.050009) (width 0.25) (layer F.Cu) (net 3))
 (segment (start 37.3 53.68483) (end 37.3 53.1) (width 0.25) (layer B.Cu) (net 3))
 (segment (start 35.671414 55.313416) (end 37.3 53.68483) (width 0.25) (layer B.Cu) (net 3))
 (segment (start 40.3 53.534104) (end 40.3 53.1) (width 0.25) (layer B.Cu) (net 3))
 (segment (start 42.079312 55.313416) (end 40.3 53.534104) (width 0.25) (layer B.Cu) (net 3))
 (via (at 43.8 35.2) (size 0.8) (drill 0.4) (layers F.Cu B.Cu) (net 10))
 (segment (start 38.16 40.84) (end 43.8 35.2) (width 0.25) (layer B.Cu) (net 10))
 (segment (start 35.075363 40.84) (end 38.16 40.84) (width 0.25) (layer B.Cu) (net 10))
 (segment (start 43.8 34.472728) (end 46.875363 31.397365) (width 0.25) (layer F.Cu) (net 10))
 (segment (start 43.8 35.2) (end 43.8 34.472728) (width 0.25) (layer F.Cu) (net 10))
 (segment (start 46.075364 50.717366) (end 46.017366 50.717366) (width 0.25) (layer B.Cu) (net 11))
 (segment (start 46.875363 51.517365) (end 46.075364 50.717366) (width 0.25) (layer B.Cu) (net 11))
 (segment (start 46.017366 50.717366) (end 43.1 47.8) (width 0.25) (layer B.Cu) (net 11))
 (via (at 43.1 47.8) (size 0.8) (drill 0.4) (layers F.Cu B.Cu) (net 11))
 (segment (start 39.3 38.3) (end 35.075363 38.3) (width 0.25) (layer F.Cu) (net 11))
 (segment (start 41.2 40.2) (end 39.3 38.3) (width 0.25) (layer F.Cu) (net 11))
 (segment (start 41.2 46.465685) (end 41.2 40.2) (width 0.25) (layer F.Cu) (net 11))
 (segment (start 42.534315 47.8) (end 41.2 46.465685) (width 0.25) (layer F.Cu) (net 11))
 (segment (start 43.1 47.8) (end 42.534315 47.8) (width 0.25) (layer F.Cu) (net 11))
 (segment (start 42.695363 37.895363) (end 42.695363 38.3) (width 0.25) (layer F.Cu) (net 6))
 (segment (start 38.9 34.1) (end 42.695363 37.895363) (width 0.25) (layer F.Cu) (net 6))
 (segment (start 46.875363 42.48) (end 46.875363 43.897365) (width 0.25) (layer F.Cu) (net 6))
 (segment (start 42.695363 38.3) (end 46.875363 42.48) (width 0.25) (layer F.Cu) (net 6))
 (segment (start 37.540363 29.517365) (end 38.875363 29.517365) (width 0.25) (layer F.Cu) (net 12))
 (segment (start 36.36 32.85) (end 36.36 34.1) (width 0.25) (layer F.Cu) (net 12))
 (segment (start 36.36 30.347597) (end 36.36 32.85) (width 0.25) (layer F.Cu) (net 12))
 (segment (start 37.107597 29.6) (end 36.36 30.347597) (width 0.25) (layer F.Cu) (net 12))
 (segment (start 38.875363 29.6) (end 37.107597 29.6) (width 0.25) (layer F.Cu) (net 12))
 (segment (start 38.755363 49.6) (end 38.875363 49.6) (width 0.25) (layer F.Cu) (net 9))
 (segment (start 35.075363 45.92) (end 38.755363 49.6) (width 0.25) (layer F.Cu) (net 9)))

